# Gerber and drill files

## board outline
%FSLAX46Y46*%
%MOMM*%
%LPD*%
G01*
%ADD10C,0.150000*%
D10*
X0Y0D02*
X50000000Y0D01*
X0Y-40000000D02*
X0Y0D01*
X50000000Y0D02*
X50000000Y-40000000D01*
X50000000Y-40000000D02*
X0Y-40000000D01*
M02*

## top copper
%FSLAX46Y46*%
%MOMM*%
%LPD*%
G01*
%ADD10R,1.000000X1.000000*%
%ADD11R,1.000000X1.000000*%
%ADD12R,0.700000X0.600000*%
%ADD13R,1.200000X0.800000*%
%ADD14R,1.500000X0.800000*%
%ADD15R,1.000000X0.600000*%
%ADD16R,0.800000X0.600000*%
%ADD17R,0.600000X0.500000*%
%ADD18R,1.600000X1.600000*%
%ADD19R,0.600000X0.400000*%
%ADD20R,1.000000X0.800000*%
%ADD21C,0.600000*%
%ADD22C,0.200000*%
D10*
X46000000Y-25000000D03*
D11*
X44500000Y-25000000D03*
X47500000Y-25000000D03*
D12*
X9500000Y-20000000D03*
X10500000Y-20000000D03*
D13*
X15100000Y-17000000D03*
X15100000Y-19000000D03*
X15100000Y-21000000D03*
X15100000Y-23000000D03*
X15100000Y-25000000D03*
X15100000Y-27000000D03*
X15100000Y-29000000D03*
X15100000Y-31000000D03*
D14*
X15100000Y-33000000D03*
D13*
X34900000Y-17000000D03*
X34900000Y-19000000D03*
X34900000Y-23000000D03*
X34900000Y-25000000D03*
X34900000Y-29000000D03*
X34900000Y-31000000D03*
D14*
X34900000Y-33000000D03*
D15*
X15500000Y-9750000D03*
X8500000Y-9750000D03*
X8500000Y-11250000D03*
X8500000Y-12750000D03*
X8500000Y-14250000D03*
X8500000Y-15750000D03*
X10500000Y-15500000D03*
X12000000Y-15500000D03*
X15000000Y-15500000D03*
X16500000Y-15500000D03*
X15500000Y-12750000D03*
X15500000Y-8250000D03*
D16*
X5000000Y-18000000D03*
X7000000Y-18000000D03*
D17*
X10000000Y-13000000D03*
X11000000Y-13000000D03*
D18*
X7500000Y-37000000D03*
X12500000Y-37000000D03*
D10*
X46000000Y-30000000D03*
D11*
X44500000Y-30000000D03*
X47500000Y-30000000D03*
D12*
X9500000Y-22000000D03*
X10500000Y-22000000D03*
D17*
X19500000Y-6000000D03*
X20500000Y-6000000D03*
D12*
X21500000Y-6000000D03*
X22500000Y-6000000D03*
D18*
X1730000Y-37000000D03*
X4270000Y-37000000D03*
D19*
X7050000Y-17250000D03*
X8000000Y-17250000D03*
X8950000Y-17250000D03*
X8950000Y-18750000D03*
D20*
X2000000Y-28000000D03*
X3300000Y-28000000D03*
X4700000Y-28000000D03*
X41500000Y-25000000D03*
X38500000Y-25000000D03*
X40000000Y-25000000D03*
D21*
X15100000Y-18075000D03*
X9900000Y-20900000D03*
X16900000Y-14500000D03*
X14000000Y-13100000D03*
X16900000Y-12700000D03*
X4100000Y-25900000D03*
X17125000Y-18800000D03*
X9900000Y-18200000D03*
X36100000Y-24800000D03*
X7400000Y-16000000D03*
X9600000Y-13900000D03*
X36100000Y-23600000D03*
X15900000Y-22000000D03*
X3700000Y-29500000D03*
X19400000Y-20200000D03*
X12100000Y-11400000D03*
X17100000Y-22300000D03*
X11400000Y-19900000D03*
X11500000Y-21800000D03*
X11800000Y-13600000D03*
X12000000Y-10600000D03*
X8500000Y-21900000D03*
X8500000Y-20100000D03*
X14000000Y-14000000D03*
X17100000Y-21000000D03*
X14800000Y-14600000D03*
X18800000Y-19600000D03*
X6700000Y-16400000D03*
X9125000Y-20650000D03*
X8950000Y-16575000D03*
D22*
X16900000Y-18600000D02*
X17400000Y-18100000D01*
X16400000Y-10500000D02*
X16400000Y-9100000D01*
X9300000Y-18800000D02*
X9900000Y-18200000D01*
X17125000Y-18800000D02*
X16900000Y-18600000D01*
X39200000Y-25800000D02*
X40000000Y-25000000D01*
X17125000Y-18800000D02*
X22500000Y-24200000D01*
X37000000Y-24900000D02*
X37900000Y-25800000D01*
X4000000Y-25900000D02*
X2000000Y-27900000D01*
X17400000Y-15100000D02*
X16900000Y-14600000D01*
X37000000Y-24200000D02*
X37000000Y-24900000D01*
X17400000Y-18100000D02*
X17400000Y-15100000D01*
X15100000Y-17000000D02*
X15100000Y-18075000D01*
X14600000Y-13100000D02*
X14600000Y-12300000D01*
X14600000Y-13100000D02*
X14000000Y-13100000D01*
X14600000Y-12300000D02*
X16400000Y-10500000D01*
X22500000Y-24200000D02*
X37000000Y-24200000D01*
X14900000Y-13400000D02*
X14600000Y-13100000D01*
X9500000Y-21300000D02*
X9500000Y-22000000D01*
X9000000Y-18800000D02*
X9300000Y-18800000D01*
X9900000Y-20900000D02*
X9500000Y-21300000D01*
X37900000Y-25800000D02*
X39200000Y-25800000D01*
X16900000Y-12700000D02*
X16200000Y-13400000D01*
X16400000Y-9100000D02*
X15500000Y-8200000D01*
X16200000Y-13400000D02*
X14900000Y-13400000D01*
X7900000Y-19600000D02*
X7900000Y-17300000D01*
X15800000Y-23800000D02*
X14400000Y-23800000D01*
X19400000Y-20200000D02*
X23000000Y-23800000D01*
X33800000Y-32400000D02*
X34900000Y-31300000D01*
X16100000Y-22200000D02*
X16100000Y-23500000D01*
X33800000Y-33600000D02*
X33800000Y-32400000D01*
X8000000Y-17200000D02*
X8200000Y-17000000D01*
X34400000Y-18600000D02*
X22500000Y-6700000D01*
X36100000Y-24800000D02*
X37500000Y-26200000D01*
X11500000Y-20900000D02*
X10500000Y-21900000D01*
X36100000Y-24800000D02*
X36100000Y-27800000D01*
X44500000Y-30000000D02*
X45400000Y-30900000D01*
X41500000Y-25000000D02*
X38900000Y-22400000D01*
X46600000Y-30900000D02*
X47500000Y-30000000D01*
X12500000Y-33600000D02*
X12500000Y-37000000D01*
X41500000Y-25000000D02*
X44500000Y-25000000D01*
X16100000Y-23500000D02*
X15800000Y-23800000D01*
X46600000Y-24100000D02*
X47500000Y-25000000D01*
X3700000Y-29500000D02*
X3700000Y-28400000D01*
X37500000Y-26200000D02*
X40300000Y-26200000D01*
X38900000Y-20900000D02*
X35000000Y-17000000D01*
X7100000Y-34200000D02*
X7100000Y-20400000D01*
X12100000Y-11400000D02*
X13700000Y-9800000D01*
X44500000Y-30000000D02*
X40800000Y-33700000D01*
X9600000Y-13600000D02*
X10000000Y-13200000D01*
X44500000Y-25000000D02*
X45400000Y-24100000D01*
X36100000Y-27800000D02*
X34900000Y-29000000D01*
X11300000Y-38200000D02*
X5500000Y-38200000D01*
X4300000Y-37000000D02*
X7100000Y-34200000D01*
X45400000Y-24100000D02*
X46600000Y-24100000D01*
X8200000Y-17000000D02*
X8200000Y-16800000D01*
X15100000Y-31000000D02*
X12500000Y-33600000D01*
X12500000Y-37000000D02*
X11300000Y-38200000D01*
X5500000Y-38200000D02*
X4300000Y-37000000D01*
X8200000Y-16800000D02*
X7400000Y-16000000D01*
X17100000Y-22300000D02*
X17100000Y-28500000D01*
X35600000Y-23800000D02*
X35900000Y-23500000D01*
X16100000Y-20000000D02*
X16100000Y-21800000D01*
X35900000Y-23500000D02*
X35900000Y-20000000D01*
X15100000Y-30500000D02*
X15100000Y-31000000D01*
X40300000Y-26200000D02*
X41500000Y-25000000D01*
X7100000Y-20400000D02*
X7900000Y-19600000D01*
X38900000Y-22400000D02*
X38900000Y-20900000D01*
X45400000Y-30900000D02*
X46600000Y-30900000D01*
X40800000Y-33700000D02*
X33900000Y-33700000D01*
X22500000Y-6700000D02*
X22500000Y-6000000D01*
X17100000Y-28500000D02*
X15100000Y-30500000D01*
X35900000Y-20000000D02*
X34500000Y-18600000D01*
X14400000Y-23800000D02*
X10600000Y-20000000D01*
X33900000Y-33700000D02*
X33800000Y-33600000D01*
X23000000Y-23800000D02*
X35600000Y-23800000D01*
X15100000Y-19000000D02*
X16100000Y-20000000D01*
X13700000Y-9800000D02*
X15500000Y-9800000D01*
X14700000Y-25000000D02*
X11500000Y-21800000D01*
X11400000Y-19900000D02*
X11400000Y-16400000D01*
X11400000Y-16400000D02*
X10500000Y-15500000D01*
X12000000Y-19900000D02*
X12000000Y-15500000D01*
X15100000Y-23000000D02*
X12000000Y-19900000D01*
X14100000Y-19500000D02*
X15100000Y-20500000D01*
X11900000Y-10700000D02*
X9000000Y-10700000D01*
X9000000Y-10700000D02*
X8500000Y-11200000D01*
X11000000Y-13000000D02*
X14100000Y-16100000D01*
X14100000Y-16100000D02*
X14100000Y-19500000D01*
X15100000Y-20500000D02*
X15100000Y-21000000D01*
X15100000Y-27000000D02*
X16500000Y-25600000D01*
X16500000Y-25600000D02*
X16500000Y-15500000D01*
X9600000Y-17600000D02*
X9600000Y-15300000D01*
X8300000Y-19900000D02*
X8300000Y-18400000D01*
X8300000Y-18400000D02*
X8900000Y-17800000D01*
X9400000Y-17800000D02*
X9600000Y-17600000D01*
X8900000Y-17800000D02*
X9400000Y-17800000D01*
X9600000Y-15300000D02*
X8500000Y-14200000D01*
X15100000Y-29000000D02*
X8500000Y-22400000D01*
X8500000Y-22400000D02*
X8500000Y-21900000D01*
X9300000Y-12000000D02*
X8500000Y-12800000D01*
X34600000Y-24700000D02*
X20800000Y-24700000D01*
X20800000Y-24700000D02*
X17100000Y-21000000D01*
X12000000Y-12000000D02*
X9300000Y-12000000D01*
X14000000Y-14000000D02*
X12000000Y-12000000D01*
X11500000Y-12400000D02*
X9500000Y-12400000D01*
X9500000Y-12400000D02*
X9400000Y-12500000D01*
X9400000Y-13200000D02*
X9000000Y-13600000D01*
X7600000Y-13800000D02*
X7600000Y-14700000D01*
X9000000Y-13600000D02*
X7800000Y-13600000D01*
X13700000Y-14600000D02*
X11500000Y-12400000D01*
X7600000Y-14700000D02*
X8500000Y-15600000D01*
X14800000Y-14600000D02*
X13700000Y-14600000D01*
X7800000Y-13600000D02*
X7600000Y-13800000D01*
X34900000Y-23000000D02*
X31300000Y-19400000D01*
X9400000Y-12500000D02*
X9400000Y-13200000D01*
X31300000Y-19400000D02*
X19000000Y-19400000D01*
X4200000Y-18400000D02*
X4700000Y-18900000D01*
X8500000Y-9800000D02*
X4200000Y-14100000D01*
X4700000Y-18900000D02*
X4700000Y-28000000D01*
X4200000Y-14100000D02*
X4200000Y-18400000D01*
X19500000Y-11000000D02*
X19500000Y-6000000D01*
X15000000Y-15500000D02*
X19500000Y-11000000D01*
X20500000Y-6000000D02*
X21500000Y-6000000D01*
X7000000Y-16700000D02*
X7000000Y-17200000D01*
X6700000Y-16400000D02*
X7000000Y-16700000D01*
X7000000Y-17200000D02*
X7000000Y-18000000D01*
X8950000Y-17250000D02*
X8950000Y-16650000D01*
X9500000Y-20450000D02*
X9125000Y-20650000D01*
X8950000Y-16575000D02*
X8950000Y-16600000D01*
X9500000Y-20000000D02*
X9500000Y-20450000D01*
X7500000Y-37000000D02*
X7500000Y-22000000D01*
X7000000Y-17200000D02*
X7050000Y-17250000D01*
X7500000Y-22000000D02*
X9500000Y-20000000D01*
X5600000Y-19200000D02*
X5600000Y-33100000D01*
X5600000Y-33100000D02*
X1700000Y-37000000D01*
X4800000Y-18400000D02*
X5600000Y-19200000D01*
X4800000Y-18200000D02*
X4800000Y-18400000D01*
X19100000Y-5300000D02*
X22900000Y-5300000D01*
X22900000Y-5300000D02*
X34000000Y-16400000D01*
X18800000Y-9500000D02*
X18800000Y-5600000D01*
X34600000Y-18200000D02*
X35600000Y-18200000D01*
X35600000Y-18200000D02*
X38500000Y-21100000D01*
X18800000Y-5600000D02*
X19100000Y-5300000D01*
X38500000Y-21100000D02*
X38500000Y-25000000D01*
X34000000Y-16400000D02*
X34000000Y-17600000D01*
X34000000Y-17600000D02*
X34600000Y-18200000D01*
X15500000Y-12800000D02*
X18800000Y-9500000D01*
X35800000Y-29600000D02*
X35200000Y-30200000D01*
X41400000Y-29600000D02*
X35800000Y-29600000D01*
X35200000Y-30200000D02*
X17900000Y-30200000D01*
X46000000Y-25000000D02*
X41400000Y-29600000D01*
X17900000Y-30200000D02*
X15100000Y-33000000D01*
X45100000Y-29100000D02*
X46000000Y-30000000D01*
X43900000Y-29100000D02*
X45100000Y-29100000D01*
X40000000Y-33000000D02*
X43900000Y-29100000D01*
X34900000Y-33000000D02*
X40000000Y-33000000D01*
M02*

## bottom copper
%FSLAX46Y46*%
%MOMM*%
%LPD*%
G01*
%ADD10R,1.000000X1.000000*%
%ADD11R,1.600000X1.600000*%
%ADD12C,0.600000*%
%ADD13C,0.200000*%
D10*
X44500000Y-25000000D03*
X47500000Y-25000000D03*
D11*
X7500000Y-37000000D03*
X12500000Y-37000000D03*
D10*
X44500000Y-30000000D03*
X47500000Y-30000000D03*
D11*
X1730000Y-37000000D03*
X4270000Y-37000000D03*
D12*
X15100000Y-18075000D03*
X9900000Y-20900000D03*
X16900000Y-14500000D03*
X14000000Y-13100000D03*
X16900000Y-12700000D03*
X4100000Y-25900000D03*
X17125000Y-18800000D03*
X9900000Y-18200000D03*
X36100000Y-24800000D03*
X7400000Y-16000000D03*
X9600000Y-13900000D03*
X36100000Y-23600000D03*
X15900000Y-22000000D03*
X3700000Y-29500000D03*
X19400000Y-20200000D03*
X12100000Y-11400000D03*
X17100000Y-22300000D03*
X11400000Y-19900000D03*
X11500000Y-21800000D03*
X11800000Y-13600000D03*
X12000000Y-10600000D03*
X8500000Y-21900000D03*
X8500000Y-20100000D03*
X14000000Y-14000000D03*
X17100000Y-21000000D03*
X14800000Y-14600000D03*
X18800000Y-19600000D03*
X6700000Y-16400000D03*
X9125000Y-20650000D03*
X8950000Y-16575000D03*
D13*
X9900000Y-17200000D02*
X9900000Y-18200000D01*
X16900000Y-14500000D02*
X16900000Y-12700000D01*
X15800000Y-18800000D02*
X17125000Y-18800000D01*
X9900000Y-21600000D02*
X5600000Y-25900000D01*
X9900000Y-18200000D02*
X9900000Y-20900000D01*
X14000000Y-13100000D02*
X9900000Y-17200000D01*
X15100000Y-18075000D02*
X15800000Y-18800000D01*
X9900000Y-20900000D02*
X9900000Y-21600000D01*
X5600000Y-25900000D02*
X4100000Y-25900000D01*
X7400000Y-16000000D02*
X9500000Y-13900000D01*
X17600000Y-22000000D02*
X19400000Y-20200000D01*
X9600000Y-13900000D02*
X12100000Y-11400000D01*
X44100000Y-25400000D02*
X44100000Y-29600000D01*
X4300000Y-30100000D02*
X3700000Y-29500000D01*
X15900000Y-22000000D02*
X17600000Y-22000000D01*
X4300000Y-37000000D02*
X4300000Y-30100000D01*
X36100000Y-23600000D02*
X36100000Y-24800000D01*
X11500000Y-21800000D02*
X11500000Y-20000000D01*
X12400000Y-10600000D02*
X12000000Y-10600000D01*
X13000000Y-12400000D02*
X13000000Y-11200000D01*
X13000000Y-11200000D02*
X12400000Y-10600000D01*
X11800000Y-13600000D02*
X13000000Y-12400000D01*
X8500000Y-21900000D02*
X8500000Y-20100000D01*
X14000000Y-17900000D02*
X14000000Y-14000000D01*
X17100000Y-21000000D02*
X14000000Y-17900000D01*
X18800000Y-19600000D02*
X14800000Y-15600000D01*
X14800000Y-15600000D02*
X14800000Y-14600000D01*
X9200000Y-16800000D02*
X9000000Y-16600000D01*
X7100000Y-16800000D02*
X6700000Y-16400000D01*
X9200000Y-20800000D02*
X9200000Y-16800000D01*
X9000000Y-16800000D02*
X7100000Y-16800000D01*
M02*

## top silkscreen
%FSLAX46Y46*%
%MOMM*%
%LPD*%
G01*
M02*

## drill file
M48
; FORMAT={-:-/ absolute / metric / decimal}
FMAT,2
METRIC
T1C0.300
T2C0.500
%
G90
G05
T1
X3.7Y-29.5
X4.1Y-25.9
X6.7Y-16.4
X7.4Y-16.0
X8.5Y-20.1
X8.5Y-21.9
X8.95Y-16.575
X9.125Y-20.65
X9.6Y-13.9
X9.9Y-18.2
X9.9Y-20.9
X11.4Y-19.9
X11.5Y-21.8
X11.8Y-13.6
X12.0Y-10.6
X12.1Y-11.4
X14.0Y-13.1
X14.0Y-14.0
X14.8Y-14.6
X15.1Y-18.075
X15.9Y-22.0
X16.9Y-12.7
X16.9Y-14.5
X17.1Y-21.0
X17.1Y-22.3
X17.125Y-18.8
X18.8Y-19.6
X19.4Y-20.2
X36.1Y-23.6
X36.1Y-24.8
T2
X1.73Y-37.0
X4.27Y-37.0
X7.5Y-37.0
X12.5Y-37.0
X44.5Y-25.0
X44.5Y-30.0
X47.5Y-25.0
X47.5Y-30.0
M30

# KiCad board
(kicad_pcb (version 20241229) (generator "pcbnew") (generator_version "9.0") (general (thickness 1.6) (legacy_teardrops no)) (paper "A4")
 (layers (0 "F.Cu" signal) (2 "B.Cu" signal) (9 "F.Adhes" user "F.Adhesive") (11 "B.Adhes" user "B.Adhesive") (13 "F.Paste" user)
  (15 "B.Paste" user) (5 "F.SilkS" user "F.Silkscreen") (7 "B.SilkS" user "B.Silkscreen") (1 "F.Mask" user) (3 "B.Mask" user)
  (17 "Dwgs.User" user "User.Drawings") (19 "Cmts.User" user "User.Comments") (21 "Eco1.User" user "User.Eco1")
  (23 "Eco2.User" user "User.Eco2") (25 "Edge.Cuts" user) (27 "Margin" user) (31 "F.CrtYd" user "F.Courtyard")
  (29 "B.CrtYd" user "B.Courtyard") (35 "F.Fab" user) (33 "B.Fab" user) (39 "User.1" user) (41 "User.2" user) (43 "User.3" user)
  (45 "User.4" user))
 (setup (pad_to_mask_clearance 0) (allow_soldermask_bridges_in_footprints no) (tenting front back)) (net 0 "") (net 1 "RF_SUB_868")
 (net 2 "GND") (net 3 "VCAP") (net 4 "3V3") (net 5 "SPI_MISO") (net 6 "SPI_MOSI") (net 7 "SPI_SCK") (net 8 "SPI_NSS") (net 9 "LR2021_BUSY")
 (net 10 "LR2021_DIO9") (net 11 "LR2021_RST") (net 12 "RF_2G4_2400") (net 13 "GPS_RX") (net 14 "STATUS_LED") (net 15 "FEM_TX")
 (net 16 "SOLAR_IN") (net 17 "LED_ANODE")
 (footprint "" (layer "F.Cu") (at 46 25)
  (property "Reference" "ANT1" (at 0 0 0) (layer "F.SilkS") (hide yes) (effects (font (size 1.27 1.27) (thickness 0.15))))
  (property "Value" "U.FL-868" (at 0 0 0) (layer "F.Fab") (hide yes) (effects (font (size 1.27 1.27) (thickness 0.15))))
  (pad "1" smd rect (at 0 0) (size 1 1) (layers "F.Cu" "F.Mask") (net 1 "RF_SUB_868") (thermal_bridge_angle 45))
  (pad "2" thru_hole rect (at -1.5 0) (size 1 1) (drill 0.5) (layers "*.Cu" "*.Mask") (remove_unused_layers no) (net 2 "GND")
   (thermal_bridge_angle 45))
  (pad "3" thru_hole rect (at 1.5 0) (size 1 1) (drill 0.5) (layers "*.Cu" "*.Mask") (remove_unused_layers no) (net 2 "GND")
   (thermal_bridge_angle 45)))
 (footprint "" (layer "F.Cu") (at 10 20)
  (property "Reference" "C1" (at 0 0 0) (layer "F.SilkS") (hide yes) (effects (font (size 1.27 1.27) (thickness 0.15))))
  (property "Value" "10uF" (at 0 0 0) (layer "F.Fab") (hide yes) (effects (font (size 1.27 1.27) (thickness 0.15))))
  (pad "1" smd rect (at -0.5 0) (size 0.7 0.6) (layers "F.Cu" "F.Mask") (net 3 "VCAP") (thermal_bridge_angle 45))
  (pad "2" smd rect (at 0.5 0) (size 0.7 0.6) (layers "F.Cu" "F.Mask") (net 2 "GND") (thermal_bridge_angle 45)))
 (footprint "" (layer "F.Cu") (at 25 25)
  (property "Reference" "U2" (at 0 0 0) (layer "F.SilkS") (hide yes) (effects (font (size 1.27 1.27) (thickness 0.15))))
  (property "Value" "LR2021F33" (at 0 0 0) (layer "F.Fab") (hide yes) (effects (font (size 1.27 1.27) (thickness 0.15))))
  (pad "1" smd rect (at -9.9 -8) (size 1.2 0.8) (layers "F.Cu" "F.Mask") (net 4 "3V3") (thermal_bridge_angle 45))
  (pad "2" smd rect (at -9.9 -6) (size 1.2 0.8) (layers "F.Cu" "F.Mask") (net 2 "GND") (thermal_bridge_angle 45))
  (pad "3" smd rect (at -9.9 -4) (size 1.2 0.8) (layers "F.Cu" "F.Mask") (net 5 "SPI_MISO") (thermal_bridge_angle 45))
  (pad "4" smd rect (at -9.9 -2) (size 1.2 0.8) (layers "F.Cu" "F.Mask") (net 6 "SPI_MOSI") (thermal_bridge_angle 45))
  (pad "5" smd rect (at -9.9 0) (size 1.2 0.8) (layers "F.Cu" "F.Mask") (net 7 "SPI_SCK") (thermal_bridge_angle 45))
  (pad "6" smd rect (at -9.9 2) (size 1.2 0.8) (layers "F.Cu" "F.Mask") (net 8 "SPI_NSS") (thermal_bridge_angle 45))
  (pad "7" smd rect (at -9.9 4) (size 1.2 0.8) (layers "F.Cu" "F.Mask") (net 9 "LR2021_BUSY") (thermal_bridge_angle 45))
  (pad "8" smd rect (at -9.9 6) (size 1.2 0.8) (layers "F.Cu" "F.Mask") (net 2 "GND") (thermal_bridge_angle 45))
  (pad "9" smd rect (at -9.9 8) (size 1.5 0.8) (layers "F.Cu" "F.Mask") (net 1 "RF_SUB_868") (thermal_bridge_angle 45))
  (pad "10" smd rect (at 9.9 -8) (size 1.2 0.8) (layers "F.Cu" "F.Mask") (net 2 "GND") (thermal_bridge_angle 45))
  (pad "11" smd rect (at 9.9 -6) (size 1.2 0.8) (layers "F.Cu" "F.Mask") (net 2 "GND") (thermal_bridge_angle 45))
  (pad "13" smd rect (at 9.9 -2) (size 1.2 0.8) (layers "F.Cu" "F.Mask") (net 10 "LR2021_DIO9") (thermal_bridge_angle 45))
  (pad "14" smd rect (at 9.9 0) (size 1.2 0.8) (layers "F.Cu" "F.Mask") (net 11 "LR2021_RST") (thermal_bridge_angle 45))
  (pad "16" smd rect (at 9.9 4) (size 1.2 0.8) (layers "F.Cu" "F.Mask") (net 2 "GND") (thermal_bridge_angle 45))
  (pad "17" smd rect (at 9.9 6) (size 1.2 0.8) (layers "F.Cu" "F.Mask") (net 2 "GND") (thermal_bridge_angle 45))
  (pad "18" smd rect (at 9.9 8) (size 1.5 0.8) (layers "F.Cu" "F.Mask") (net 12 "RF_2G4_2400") (thermal_bridge_angle 45)))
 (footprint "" (layer "F.Cu") (at 12 12)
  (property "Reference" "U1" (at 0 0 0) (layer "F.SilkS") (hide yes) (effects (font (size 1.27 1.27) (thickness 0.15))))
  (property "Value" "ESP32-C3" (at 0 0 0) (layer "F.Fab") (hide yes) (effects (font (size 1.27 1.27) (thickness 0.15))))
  (pad "GND" smd rect (at 3.5 -2.25) (size 1 0.6) (layers "F.Cu" "F.Mask") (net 2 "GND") (thermal_bridge_angle 45))
  (pad "GPIO1" smd rect (at -3.5 -2.25) (size 1 0.6) (layers "F.Cu" "F.Mask") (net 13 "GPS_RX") (thermal_bridge_angle 45))
  (pad "GPIO2" smd rect (at -3.5 -0.75) (size 1 0.6) (layers "F.Cu" "F.Mask") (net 5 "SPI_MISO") (thermal_bridge_angle 45))
  (pad "GPIO3" smd rect (at -3.5 0.75) (size 1 0.6) (layers "F.Cu" "F.Mask") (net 11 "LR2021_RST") (thermal_bridge_angle 45))
  (pad "GPIO4" smd rect (at -3.5 2.25) (size 1 0.6) (layers "F.Cu" "F.Mask") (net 9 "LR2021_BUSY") (thermal_bridge_angle 45))
  (pad "GPIO5" smd rect (at -3.5 3.75) (size 1 0.6) (layers "F.Cu" "F.Mask") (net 10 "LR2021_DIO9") (thermal_bridge_angle 45))
  (pad "GPIO6" smd rect (at -1.5 3.5) (size 1 0.6) (layers "F.Cu" "F.Mask") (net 7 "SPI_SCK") (thermal_bridge_angle 45))
  (pad "GPIO7" smd rect (at 0 3.5) (size 1 0.6) (layers "F.Cu" "F.Mask") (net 6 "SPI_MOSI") (thermal_bridge_angle 45))
  (pad "GPIO9" smd rect (at 3 3.5) (size 1 0.6) (layers "F.Cu" "F.Mask") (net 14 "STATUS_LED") (thermal_bridge_angle 45))
  (pad "GPIO10" smd rect (at 4.5 3.5) (size 1 0.6) (layers "F.Cu" "F.Mask") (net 8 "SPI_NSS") (thermal_bridge_angle 45))
  (pad "GPIO19" smd rect (at 3.5 0.75) (size 1 0.6) (layers "F.Cu" "F.Mask") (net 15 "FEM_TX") (thermal_bridge_angle 45))
  (pad "VCC" smd rect (at 3.5 -3.75) (size 1 0.6) (layers "F.Cu" "F.Mask") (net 4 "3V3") (thermal_bridge_angle 45)))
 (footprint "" (layer "F.Cu") (at 6 18)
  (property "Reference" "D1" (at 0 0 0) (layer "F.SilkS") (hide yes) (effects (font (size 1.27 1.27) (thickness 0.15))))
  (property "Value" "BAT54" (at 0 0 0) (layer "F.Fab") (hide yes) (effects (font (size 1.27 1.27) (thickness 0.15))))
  (pad "A" smd rect (at -1 0) (size 0.8 0.6) (layers "F.Cu" "F.Mask") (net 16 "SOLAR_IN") (thermal_bridge_angle 45))
  (pad "K" smd rect (at 1 0) (size 0.8 0.6) (layers "F.Cu" "F.Mask") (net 3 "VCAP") (thermal_bridge_angle 45)))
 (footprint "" (layer "F.Cu") (at 10.5 13)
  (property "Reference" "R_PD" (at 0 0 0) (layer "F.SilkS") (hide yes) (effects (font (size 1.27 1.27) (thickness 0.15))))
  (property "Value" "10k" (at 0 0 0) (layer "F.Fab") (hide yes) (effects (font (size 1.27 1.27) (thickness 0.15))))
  (pad "1" smd rect (at -0.5 0) (size 0.6 0.5) (layers "F.Cu" "F.Mask") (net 2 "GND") (thermal_bridge_angle 45))
  (pad "2" smd rect (at 0.5 0) (size 0.6 0.5) (layers "F.Cu" "F.Mask") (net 5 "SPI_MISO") (thermal_bridge_angle 45)))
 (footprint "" (layer "F.Cu") (at 10 37)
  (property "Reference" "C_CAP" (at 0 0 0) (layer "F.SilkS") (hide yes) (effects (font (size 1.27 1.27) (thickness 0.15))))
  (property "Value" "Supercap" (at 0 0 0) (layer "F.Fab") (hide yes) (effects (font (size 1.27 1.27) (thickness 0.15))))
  (pad "1" thru_hole rect (at -2.5 0) (size 1.6 1.6) (drill 0.5) (layers "*.Cu" "*.Mask") (remove_unused_layers no) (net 3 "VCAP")
   (thermal_bridge_angle 45))
  (pad "2" thru_hole rect (at 2.5 0) (size 1.6 1.6) (drill 0.5) (layers "*.Cu" "*.Mask") (remove_unused_layers no) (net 2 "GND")
   (thermal_bridge_angle 45)))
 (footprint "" (layer "F.Cu") (at 46 30)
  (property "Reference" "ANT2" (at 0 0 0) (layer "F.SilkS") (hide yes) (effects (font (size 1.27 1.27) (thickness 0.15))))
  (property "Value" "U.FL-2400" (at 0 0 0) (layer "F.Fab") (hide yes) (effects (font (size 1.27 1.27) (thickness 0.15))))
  (pad "1" smd rect (at 0 0) (size 1 1) (layers "F.Cu" "F.Mask") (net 12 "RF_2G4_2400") (thermal_bridge_angle 45))
  (pad "2" thru_hole rect (at -1.5 0) (size 1 1) (drill 0.5) (layers "*.Cu" "*.Mask") (remove_unused_layers no) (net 2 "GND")
   (thermal_bridge_angle 45))
  (pad "3" thru_hole rect (at 1.5 0) (size 1 1) (drill 0.5) (layers "*.Cu" "*.Mask") (remove_unused_layers no) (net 2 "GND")
   (thermal_bridge_angle 45)))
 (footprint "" (layer "F.Cu") (at 10 22)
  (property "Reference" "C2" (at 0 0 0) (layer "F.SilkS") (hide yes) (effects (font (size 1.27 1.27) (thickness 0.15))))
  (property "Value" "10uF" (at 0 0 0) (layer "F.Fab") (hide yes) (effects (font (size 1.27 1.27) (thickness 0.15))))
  (pad "1" smd rect (at -0.5 0) (size 0.7 0.6) (layers "F.Cu" "F.Mask") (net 4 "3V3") (thermal_bridge_angle 45))
  (pad "2" smd rect (at 0.5 0) (size 0.7 0.6) (layers "F.Cu" "F.Mask") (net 2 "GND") (thermal_bridge_angle 45)))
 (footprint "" (layer "F.Cu") (at 20 6)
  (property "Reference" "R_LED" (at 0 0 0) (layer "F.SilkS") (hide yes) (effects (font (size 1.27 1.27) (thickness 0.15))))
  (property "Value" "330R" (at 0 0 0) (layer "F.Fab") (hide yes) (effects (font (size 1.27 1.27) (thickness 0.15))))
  (pad "1" smd rect (at -0.5 0) (size 0.6 0.5) (layers "F.Cu" "F.Mask") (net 14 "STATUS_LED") (thermal_bridge_angle 45))
  (pad "2" smd rect (at 0.5 0) (size 0.6 0.5) (layers "F.Cu" "F.Mask") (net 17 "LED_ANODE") (thermal_bridge_angle 45)))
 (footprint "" (layer "F.Cu") (at 22 6)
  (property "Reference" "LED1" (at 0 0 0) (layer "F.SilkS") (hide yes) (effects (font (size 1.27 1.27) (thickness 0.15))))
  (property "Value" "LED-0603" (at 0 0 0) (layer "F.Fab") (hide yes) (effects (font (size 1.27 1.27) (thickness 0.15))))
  (pad "A" smd rect (at -0.5 0) (size 0.7 0.6) (layers "F.Cu" "F.Mask") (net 17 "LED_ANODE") (thermal_bridge_angle 45))
  (pad "K" smd rect (at 0.5 0) (size 0.7 0.6) (layers "F.Cu" "F.Mask") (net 2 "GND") (thermal_bridge_angle 45)))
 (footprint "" (layer "F.Cu") (at 3 37)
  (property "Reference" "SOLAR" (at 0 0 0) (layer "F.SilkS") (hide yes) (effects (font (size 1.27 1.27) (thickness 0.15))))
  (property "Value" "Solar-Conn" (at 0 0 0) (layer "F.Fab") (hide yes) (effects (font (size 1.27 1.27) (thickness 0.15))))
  (pad "1" thru_hole rect (at -1.27 0) (size 1.6 1.6) (drill 0.5) (layers "*.Cu" "*.Mask") (remove_unused_layers no) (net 16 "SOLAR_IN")
   (thermal_bridge_angle 45))
  (pad "2" thru_hole rect (at 1.27 0) (size 1.6 1.6) (drill 0.5) (layers "*.Cu" "*.Mask") (remove_unused_layers no) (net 2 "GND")
   (thermal_bridge_angle 45)))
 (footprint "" (layer "F.Cu") (at 8 18)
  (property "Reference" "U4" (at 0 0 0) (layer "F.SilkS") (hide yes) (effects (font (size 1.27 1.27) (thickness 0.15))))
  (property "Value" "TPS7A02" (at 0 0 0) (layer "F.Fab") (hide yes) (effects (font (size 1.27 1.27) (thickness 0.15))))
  (pad "1" smd rect (at -0.95 -0.75) (size 0.6 0.4) (layers "F.Cu" "F.Mask") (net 3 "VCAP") (thermal_bridge_angle 45))
  (pad "2" smd rect (at 0 -0.75) (size 0.6 0.4) (layers "F.Cu" "F.Mask") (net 2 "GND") (thermal_bridge_angle 45))
  (pad "3" smd rect (at 0.95 -0.75) (size 0.6 0.4) (layers "F.Cu" "F.Mask") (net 3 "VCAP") (thermal_bridge_angle 45))
  (pad "4" smd rect (at 0.95 0.75) (size 0.6 0.4) (layers "F.Cu" "F.Mask") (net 4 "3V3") (thermal_bridge_angle 45)))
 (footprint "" (layer "F.Cu") (at 4 28)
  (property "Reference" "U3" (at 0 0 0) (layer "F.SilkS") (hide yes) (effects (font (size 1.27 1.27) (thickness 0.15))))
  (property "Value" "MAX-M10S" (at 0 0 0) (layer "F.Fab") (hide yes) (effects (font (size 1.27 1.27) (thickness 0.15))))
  (pad "1" smd rect (at -2 0) (size 1 0.8) (layers "F.Cu" "F.Mask") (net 4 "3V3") (thermal_bridge_angle 45))
  (pad "2" smd rect (at -0.7 0) (size 1 0.8) (layers "F.Cu" "F.Mask") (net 2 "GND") (thermal_bridge_angle 45))
  (pad "3" smd rect (at 0.7 0) (size 1 0.8) (layers "F.Cu" "F.Mask") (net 13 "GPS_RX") (thermal_bridge_angle 45)))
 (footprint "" (layer "F.Cu") (at 40 25)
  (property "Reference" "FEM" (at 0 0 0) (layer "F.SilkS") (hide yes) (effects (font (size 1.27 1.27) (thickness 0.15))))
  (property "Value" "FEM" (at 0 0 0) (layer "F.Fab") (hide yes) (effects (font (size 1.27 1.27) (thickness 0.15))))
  (pad "GND" smd rect (at 1.5 0) (size 1 0.8) (layers "F.Cu" "F.Mask") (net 2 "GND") (thermal_bridge_angle 45))
  (pad "TX" smd rect (at -1.5 0) (size 1 0.8) (layers "F.Cu" "F.Mask") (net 15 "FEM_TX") (thermal_bridge_angle 45))
  (pad "VCC" smd rect (at 0 0) (size 1 0.8) (layers "F.Cu" "F.Mask") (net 4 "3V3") (thermal_bridge_angle 45)))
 (gr_line (start 0 0) (end 50 0) (stroke (width 0.15) (type default)) (layer "Edge.Cuts"))
 (gr_line (start 0 40) (end 0 0) (stroke (width 0.15) (type default)) (layer "Edge.Cuts"))
 (gr_line (start 50 0) (end 50 40) (stroke (width 0.15) (type default)) (layer "Edge.Cuts"))
 (gr_line (start 50 40) (end 0 40) (stroke (width 0.15) (type default)) (layer "Edge.Cuts"))
 (segment (start 16.9 18.6) (end 17.4 18.1) (width 0.2) (layer "F.Cu") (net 4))
 (segment (start 16.4 10.5) (end 16.4 9.1) (width 0.2) (layer "F.Cu") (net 4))
 (segment (start 9.3 18.8) (end 9.9 18.2) (width 0.2) (layer "F.Cu") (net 4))
 (segment (start 17.125 18.8) (end 16.9 18.6) (width 0.2) (layer "F.Cu") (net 4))
 (segment (start 39.2 25.8) (end 40 25) (width 0.2) (layer "F.Cu") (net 4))
 (segment (start 17.125 18.8) (end 22.5 24.2) (width 0.2) (layer "F.Cu") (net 4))
 (segment (start 37 24.9) (end 37.9 25.8) (width 0.2) (layer "F.Cu") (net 4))
 (segment (start 4 25.9) (end 2 27.9) (width 0.2) (layer "F.Cu") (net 4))
 (segment (start 17.4 15.1) (end 16.9 14.6) (width 0.2) (layer "F.Cu") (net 4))
 (segment (start 37 24.2) (end 37 24.9) (width 0.2) (layer "F.Cu") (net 4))
 (segment (start 17.4 18.1) (end 17.4 15.1) (width 0.2) (layer "F.Cu") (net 4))
 (segment (start 15.1 17) (end 15.1 18.075) (width 0.2) (layer "F.Cu") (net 4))
 (segment (start 14.6 13.1) (end 14.6 12.3) (width 0.2) (layer "F.Cu") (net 4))
 (segment (start 14.6 13.1) (end 14 13.1) (width 0.2) (layer "F.Cu") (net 4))
 (segment (start 14.6 12.3) (end 16.4 10.5) (width 0.2) (layer "F.Cu") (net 4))
 (segment (start 22.5 24.2) (end 37 24.2) (width 0.2) (layer "F.Cu") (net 4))
 (segment (start 14.9 13.4) (end 14.6 13.1) (width 0.2) (layer "F.Cu") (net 4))
 (segment (start 9.5 21.3) (end 9.5 22) (width 0.2) (layer "F.Cu") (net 4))
 (segment (start 9 18.8) (end 9.3 18.8) (width 0.2) (layer "F.Cu") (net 4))
 (segment (start 9.9 20.9) (end 9.5 21.3) (width 0.2) (layer "F.Cu") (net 4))
 (segment (start 37.9 25.8) (end 39.2 25.8) (width 0.2) (layer "F.Cu") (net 4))
 (segment (start 16.9 12.7) (end 16.2 13.4) (width 0.2) (layer "F.Cu") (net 4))
 (segment (start 16.4 9.1) (end 15.5 8.2) (width 0.2) (layer "F.Cu") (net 4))
 (segment (start 16.2 13.4) (end 14.9 13.4) (width 0.2) (layer "F.Cu") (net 4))
 (via (at 15.1 18.075) (size 0.6) (drill 0.3) (layers "F.Cu" "B.Cu") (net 4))
 (via (at 9.9 20.9) (size 0.6) (drill 0.3) (layers "F.Cu" "B.Cu") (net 4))
 (via (at 16.9 14.5) (size 0.6) (drill 0.3) (layers "F.Cu" "B.Cu") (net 4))
 (via (at 14 13.1) (size 0.6) (drill 0.3) (layers "F.Cu" "B.Cu") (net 4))
 (via (at 16.9 12.7) (size 0.6) (drill 0.3) (layers "F.Cu" "B.Cu") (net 4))
 (via (at 4.1 25.9) (size 0.6) (drill 0.3) (layers "F.Cu" "B.Cu") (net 4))
 (via (at 17.125 18.8) (size 0.6) (drill 0.3) (layers "F.Cu" "B.Cu") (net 4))
 (via (at 9.9 18.2) (size 0.6) (drill 0.3) (layers "F.Cu" "B.Cu") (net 4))
 (segment (start 9.9 17.2) (end 9.9 18.2) (width 0.2) (layer "B.Cu") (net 4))
 (segment (start 16.9 14.5) (end 16.9 12.7) (width 0.2) (layer "B.Cu") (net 4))
 (segment (start 15.8 18.8) (end 17.125 18.8) (width 0.2) (layer "B.Cu") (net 4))
 (segment (start 9.9 21.6) (end 5.6 25.9) (width 0.2) (layer "B.Cu") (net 4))
 (segment (start 9.9 18.2) (end 9.9 20.9) (width 0.2) (layer "B.Cu") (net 4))
 (segment (start 14 13.1) (end 9.9 17.2) (width 0.2) (layer "B.Cu") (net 4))
 (segment (start 15.1 18.075) (end 15.8 18.8) (width 0.2) (layer "B.Cu") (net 4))
 (segment (start 9.9 20.9) (end 9.9 21.6) (width 0.2) (layer "B.Cu") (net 4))
 (segment (start 5.6 25.9) (end 4.1 25.9) (width 0.2) (layer "B.Cu") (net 4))
 (segment (start 7.9 19.6) (end 7.9 17.3) (width 0.2) (layer "F.Cu") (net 2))
 (segment (start 15.8 23.8) (end 14.4 23.8) (width 0.2) (layer "F.Cu") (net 2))
 (segment (start 19.4 20.2) (end 23 23.8) (width 0.2) (layer "F.Cu") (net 2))
 (segment (start 33.8 32.4) (end 34.9 31.3) (width 0.2) (layer "F.Cu") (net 2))
 (segment (start 16.1 22.2) (end 16.1 23.5) (width 0.2) (layer "F.Cu") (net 2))
 (segment (start 33.8 33.6) (end 33.8 32.4) (width 0.2) (layer "F.Cu") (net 2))
 (segment (start 8 17.2) (end 8.2 17) (width 0.2) (layer "F.Cu") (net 2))
 (segment (start 34.4 18.6) (end 22.5 6.7) (width 0.2) (layer "F.Cu") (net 2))
 (segment (start 36.1 24.8) (end 37.5 26.2) (width 0.2) (layer "F.Cu") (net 2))
 (segment (start 11.5 20.9) (end 10.5 21.9) (width 0.2) (layer "F.Cu") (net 2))
 (segment (start 36.1 24.8) (end 36.1 27.8) (width 0.2) (layer "F.Cu") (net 2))
 (segment (start 44.5 30) (end 45.4 30.9) (width 0.2) (layer "F.Cu") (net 2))
 (segment (start 41.5 25) (end 38.9 22.4) (width 0.2) (layer "F.Cu") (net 2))
 (segment (start 46.6 30.9) (end 47.5 30) (width 0.2) (layer "F.Cu") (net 2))
 (segment (start 12.5 33.6) (end 12.5 37) (width 0.2) (layer "F.Cu") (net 2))
 (segment (start 41.5 25) (end 44.5 25) (width 0.2) (layer "F.Cu") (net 2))
 (segment (start 16.1 23.5) (end 15.8 23.8) (width 0.2) (layer "F.Cu") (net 2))
 (segment (start 46.6 24.1) (end 47.5 25) (width 0.2) (layer "F.Cu") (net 2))
 (segment (start 3.7 29.5) (end 3.7 28.4) (width 0.2) (layer "F.Cu") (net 2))
 (segment (start 37.5 26.2) (end 40.3 26.2) (width 0.2) (layer "F.Cu") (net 2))
 (segment (start 38.9 20.9) (end 35 17) (width 0.2) (layer "F.Cu") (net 2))
 (segment (start 7.1 34.2) (end 7.1 20.4) (width 0.2) (layer "F.Cu") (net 2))
 (segment (start 12.1 11.4) (end 13.7 9.8) (width 0.2) (layer "F.Cu") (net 2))
 (segment (start 44.5 30) (end 40.8 33.7) (width 0.2) (layer "F.Cu") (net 2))
 (segment (start 9.6 13.6) (end 10 13.2) (width 0.2) (layer "F.Cu") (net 2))
 (segment (start 44.5 25) (end 45.4 24.1) (width 0.2) (layer "F.Cu") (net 2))
 (segment (start 36.1 27.8) (end 34.9 29) (width 0.2) (layer "F.Cu") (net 2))
 (segment (start 11.3 38.2) (end 5.5 38.2) (width 0.2) (layer "F.Cu") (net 2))
 (segment (start 4.3 37) (end 7.1 34.2) (width 0.2) (layer "F.Cu") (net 2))
 (segment (start 45.4 24.1) (end 46.6 24.1) (width 0.2) (layer "F.Cu") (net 2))
 (segment (start 8.2 17) (end 8.2 16.8) (width 0.2) (layer "F.Cu") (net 2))
 (segment (start 15.1 31) (end 12.5 33.6) (width 0.2) (layer "F.Cu") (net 2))
 (segment (start 12.5 37) (end 11.3 38.2) (width 0.2) (layer "F.Cu") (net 2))
 (segment (start 5.5 38.2) (end 4.3 37) (width 0.2) (layer "F.Cu") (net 2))
 (segment (start 8.2 16.8) (end 7.4 16) (width 0.2) (layer "F.Cu") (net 2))
 (segment (start 17.1 22.3) (end 17.1 28.5) (width 0.2) (layer "F.Cu") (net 2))
 (segment (start 35.6 23.8) (end 35.9 23.5) (width 0.2) (layer "F.Cu") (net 2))
 (segment (start 16.1 20) (end 16.1 21.8) (width 0.2) (layer "F.Cu") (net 2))
 (segment (start 35.9 23.5) (end 35.9 20) (width 0.2) (layer "F.Cu") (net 2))
 (segment (start 15.1 30.5) (end 15.1 31) (width 0.2) (layer "F.Cu") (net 2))
 (segment (start 40.3 26.2) (end 41.5 25) (width 0.2) (layer "F.Cu") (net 2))
 (segment (start 7.1 20.4) (end 7.9 19.6) (width 0.2) (layer "F.Cu") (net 2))
 (segment (start 38.9 22.4) (end 38.9 20.9) (width 0.2) (layer "F.Cu") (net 2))
 (segment (start 45.4 30.9) (end 46.6 30.9) (width 0.2) (layer "F.Cu") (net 2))
 (segment (start 40.8 33.7) (end 33.9 33.7) (width 0.2) (layer "F.Cu") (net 2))
 (segment (start 22.5 6.7) (end 22.5 6) (width 0.2) (layer "F.Cu") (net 2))
 (segment (start 17.1 28.5) (end 15.1 30.5) (width 0.2) (layer "F.Cu") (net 2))
 (segment (start 35.9 20) (end 34.5 18.6) (width 0.2) (layer "F.Cu") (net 2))
 (segment (start 14.4 23.8) (end 10.6 20) (width 0.2) (layer "F.Cu") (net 2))
 (segment (start 33.9 33.7) (end 33.8 33.6) (width 0.2) (layer "F.Cu") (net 2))
 (segment (start 23 23.8) (end 35.6 23.8) (width 0.2) (layer "F.Cu") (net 2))
 (segment (start 15.1 19) (end 16.1 20) (width 0.2) (layer "F.Cu") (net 2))
 (segment (start 13.7 9.8) (end 15.5 9.8) (width 0.2) (layer "F.Cu") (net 2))
 (via (at 36.1 24.8) (size 0.6) (drill 0.3) (layers "F.Cu" "B.Cu") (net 2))
 (via (at 7.4 16) (size 0.6) (drill 0.3) (layers "F.Cu" "B.Cu") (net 2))
 (via (at 9.6 13.9) (size 0.6) (drill 0.3) (layers "F.Cu" "B.Cu") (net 2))
 (via (at 36.1 23.6) (size 0.6) (drill 0.3) (layers "F.Cu" "B.Cu") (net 2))
 (via (at 15.9 22) (size 0.6) (drill 0.3) (layers "F.Cu" "B.Cu") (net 2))
 (via (at 3.7 29.5) (size 0.6) (drill 0.3) (layers "F.Cu" "B.Cu") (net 2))
 (via (at 19.4 20.2) (size 0.6) (drill 0.3) (layers "F.Cu" "B.Cu") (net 2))
 (via (at 12.1 11.4) (size 0.6) (drill 0.3) (layers "F.Cu" "B.Cu") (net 2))
 (via (at 17.1 22.3) (size 0.6) (drill 0.3) (layers "F.Cu" "B.Cu") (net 2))
 (segment (start 7.4 16) (end 9.5 13.9) (width 0.2) (layer "B.Cu") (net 2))
 (segment (start 17.6 22) (end 19.4 20.2) (width 0.2) (layer "B.Cu") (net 2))
 (segment (start 9.6 13.9) (end 12.1 11.4) (width 0.2) (layer "B.Cu") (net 2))
 (segment (start 44.1 25.4) (end 44.1 29.6) (width 0.2) (layer "B.Cu") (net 2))
 (segment (start 4.3 30.1) (end 3.7 29.5) (width 0.2) (layer "B.Cu") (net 2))
 (segment (start 15.9 22) (end 17.6 22) (width 0.2) (layer "B.Cu") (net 2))
 (segment (start 4.3 37) (end 4.3 30.1) (width 0.2) (layer "B.Cu") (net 2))
 (segment (start 36.1 23.6) (end 36.1 24.8) (width 0.2) (layer "B.Cu") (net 2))
 (segment (start 14.7 25) (end 11.5 21.8) (width 0.2) (layer "F.Cu") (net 7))
 (segment (start 11.4 19.9) (end 11.4 16.4) (width 0.2) (layer "F.Cu") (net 7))
 (segment (start 11.4 16.4) (end 10.5 15.5) (width 0.2) (layer "F.Cu") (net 7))
 (via (at 11.4 19.9) (size 0.6) (drill 0.3) (layers "F.Cu" "B.Cu") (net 7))
 (via (at 11.5 21.8) (size 0.6) (drill 0.3) (layers "F.Cu" "B.Cu") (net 7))
 (segment (start 11.5 21.8) (end 11.5 20) (width 0.2) (layer "B.Cu") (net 7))
 (segment (start 12 19.9) (end 12 15.5) (width 0.2) (layer "F.Cu") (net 6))
 (segment (start 15.1 23) (end 12 19.9) (width 0.2) (layer "F.Cu") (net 6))
 (segment (start 14.1 19.5) (end 15.1 20.5) (width 0.2) (layer "F.Cu") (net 5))
 (segment (start 11.9 10.7) (end 9 10.7) (width 0.2) (layer "F.Cu") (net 5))
 (segment (start 9 10.7) (end 8.5 11.2) (width 0.2) (layer "F.Cu") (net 5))
 (segment (start 11 13) (end 14.1 16.1) (width 0.2) (layer "F.Cu") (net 5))
 (segment (start 14.1 16.1) (end 14.1 19.5) (width 0.2) (layer "F.Cu") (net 5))
 (segment (start 15.1 20.5) (end 15.1 21) (width 0.2) (layer "F.Cu") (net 5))
 (via (at 11.8 13.6) (size 0.6) (drill 0.3) (layers "F.Cu" "B.Cu") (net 5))
 (via (at 12 10.6) (size 0.6) (drill 0.3) (layers "F.Cu" "B.Cu") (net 5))
 (segment (start 12.4 10.6) (end 12 10.6) (width 0.2) (layer "B.Cu") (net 5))
 (segment (start 13 12.4) (end 13 11.2) (width 0.2) (layer "B.Cu") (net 5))
 (segment (start 13 11.2) (end 12.4 10.6) (width 0.2) (layer "B.Cu") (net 5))
 (segment (start 11.8 13.6) (end 13 12.4) (width 0.2) (layer "B.Cu") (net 5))
 (segment (start 15.1 27) (end 16.5 25.6) (width 0.2) (layer "F.Cu") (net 8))
 (segment (start 16.5 25.6) (end 16.5 15.5) (width 0.2) (layer "F.Cu") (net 8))
 (segment (start 9.6 17.6) (end 9.6 15.3) (width 0.2) (layer "F.Cu") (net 9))
 (segment (start 8.3 19.9) (end 8.3 18.4) (width 0.2) (layer "F.Cu") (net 9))
 (segment (start 8.3 18.4) (end 8.9 17.8) (width 0.2) (layer "F.Cu") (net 9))
 (segment (start 9.4 17.8) (end 9.6 17.6) (width 0.2) (layer "F.Cu") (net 9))
 (segment (start 8.9 17.8) (end 9.4 17.8) (width 0.2) (layer "F.Cu") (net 9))
 (segment (start 9.6 15.3) (end 8.5 14.2) (width 0.2) (layer "F.Cu") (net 9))
 (segment (start 15.1 29) (end 8.5 22.4) (width 0.2) (layer "F.Cu") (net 9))
 (segment (start 8.5 22.4) (end 8.5 21.9) (width 0.2) (layer "F.Cu") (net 9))
 (via (at 8.5 21.9) (size 0.6) (drill 0.3) (layers "F.Cu" "B.Cu") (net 9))
 (via (at 8.5 20.1) (size 0.6) (drill 0.3) (layers "F.Cu" "B.Cu") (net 9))
 (segment (start 8.5 21.9) (end 8.5 20.1) (width 0.2) (layer "B.Cu") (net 9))
 (segment (start 9.3 12) (end 8.5 12.8) (width 0.2) (layer "F.Cu") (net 11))
 (segment (start 34.6 24.7) (end 20.8 24.7) (width 0.2) (layer "F.Cu") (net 11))
 (segment (start 20.8 24.7) (end 17.1 21) (width 0.2) (layer "F.Cu") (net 11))
 (segment (start 12 12) (end 9.3 12) (width 0.2) (layer "F.Cu") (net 11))
 (segment (start 14 14) (end 12 12) (width 0.2) (layer "F.Cu") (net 11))
 (via (at 14 14) (size 0.6) (drill 0.3) (layers "F.Cu" "B.Cu") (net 11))
 (via (at 17.1 21) (size 0.6) (drill 0.3) (layers "F.Cu" "B.Cu") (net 11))
 (segment (start 14 17.9) (end 14 14) (width 0.2) (layer "B.Cu") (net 11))
 (segment (start 17.1 21) (end 14 17.9) (width 0.2) (layer "B.Cu") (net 11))
 (segment (start 11.5 12.4) (end 9.5 12.4) (width 0.2) (layer "F.Cu") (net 10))
 (segment (start 9.5 12.4) (end 9.4 12.5) (width 0.2) (layer "F.Cu") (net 10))
 (segment (start 9.4 13.2) (end 9 13.6) (width 0.2) (layer "F.Cu") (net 10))
 (segment (start 7.6 13.8) (end 7.6 14.7) (width 0.2) (layer "F.Cu") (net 10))
 (segment (start 9 13.6) (end 7.8 13.6) (width 0.2) (layer "F.Cu") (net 10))
 (segment (start 13.7 14.6) (end 11.5 12.4) (width 0.2) (layer "F.Cu") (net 10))
 (segment (start 7.6 14.7) (end 8.5 15.6) (width 0.2) (layer "F.Cu") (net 10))
 (segment (start 14.8 14.6) (end 13.7 14.6) (width 0.2) (layer "F.Cu") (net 10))
 (segment (start 7.8 13.6) (end 7.6 13.8) (width 0.2) (layer "F.Cu") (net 10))
 (segment (start 34.9 23) (end 31.3 19.4) (width 0.2) (layer "F.Cu") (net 10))
 (segment (start 9.4 12.5) (end 9.4 13.2) (width 0.2) (layer "F.Cu") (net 10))
 (segment (start 31.3 19.4) (end 19 19.4) (width 0.2) (layer "F.Cu") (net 10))
 (via (at 14.8 14.6) (size 0.6) (drill 0.3) (layers "F.Cu" "B.Cu") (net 10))
 (via (at 18.8 19.6) (size 0.6) (drill 0.3) (layers "F.Cu" "B.Cu") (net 10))
 (segment (start 18.8 19.6) (end 14.8 15.6) (width 0.2) (layer "B.Cu") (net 10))
 (segment (start 14.8 15.6) (end 14.8 14.6) (width 0.2) (layer "B.Cu") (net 10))
 (segment (start 4.2 18.4) (end 4.7 18.9) (width 0.2) (layer "F.Cu") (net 13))
 (segment (start 8.5 9.8) (end 4.2 14.1) (width 0.2) (layer "F.Cu") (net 13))
 (segment (start 4.7 18.9) (end 4.7 28) (width 0.2) (layer "F.Cu") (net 13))
 (segment (start 4.2 14.1) (end 4.2 18.4) (width 0.2) (layer "F.Cu") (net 13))
 (segment (start 19.5 11) (end 19.5 6) (width 0.2) (layer "F.Cu") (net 14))
 (segment (start 15 15.5) (end 19.5 11) (width 0.2) (layer "F.Cu") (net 14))
 (segment (start 20.5 6) (end 21.5 6) (width 0.2) (layer "F.Cu") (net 17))
 (segment (start 7 16.7) (end 7 17.2) (width 0.2) (layer "F.Cu") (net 3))
 (segment (start 6.7 16.4) (end 7 16.7) (width 0.2) (layer "F.Cu") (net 3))
 (segment (start 7 17.2) (end 7 18) (width 0.2) (layer "F.Cu") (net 3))
 (segment (start 8.95 17.25) (end 8.95 16.65) (width 0.2) (layer "F.Cu") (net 3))
 (segment (start 9.5 20.45) (end 9.125 20.65) (width 0.2) (layer "F.Cu") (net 3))
 (segment (start 8.95 16.575) (end 8.95 16.6) (width 0.2) (layer "F.Cu") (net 3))
 (segment (start 9.5 20) (end 9.5 20.45) (width 0.2) (layer "F.Cu") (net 3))
 (segment (start 7.5 37) (end 7.5 22) (width 0.2) (layer "F.Cu") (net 3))
 (segment (start 7 17.2) (end 7.05 17.25) (width 0.2) (layer "F.Cu") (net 3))
 (segment (start 7.5 22) (end 9.5 20) (width 0.2) (layer "F.Cu") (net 3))
 (via (at 6.7 16.4) (size 0.6) (drill 0.3) (layers "F.Cu" "B.Cu") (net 3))
 (via (at 9.125 20.65) (size 0.6) (drill 0.3) (layers "F.Cu" "B.Cu") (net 3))
 (via (at 8.95 16.575) (size 0.6) (drill 0.3) (layers "F.Cu" "B.Cu") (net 3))
 (segment (start 9.2 16.8) (end 9 16.6) (width 0.2) (layer "B.Cu") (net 3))
 (segment (start 7.1 16.8) (end 6.7 16.4) (width 0.2) (layer "B.Cu") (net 3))
 (segment (start 9.2 20.8) (end 9.2 16.8) (width 0.2) (layer "B.Cu") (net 3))
 (segment (start 9 16.8) (end 7.1 16.8) (width 0.2) (layer "B.Cu") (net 3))
 (segment (start 5.6 19.2) (end 5.6 33.1) (width 0.2) (layer "F.Cu") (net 16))
 (segment (start 5.6 33.1) (end 1.7 37) (width 0.2) (layer "F.Cu") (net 16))
 (segment (start 4.8 18.4) (end 5.6 19.2) (width 0.2) (layer "F.Cu") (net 16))
 (segment (start 4.8 18.2) (end 4.8 18.4) (width 0.2) (layer "F.Cu") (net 16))
 (segment (start 19.1 5.3) (end 22.9 5.3) (width 0.2) (layer "F.Cu") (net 15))
 (segment (start 22.9 5.3) (end 34 16.4) (width 0.2) (layer "F.Cu") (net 15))
 (segment (start 18.8 9.5) (end 18.8 5.6) (width 0.2) (layer "F.Cu") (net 15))
 (segment (start 34.6 18.2) (end 35.6 18.2) (width 0.2) (layer "F.Cu") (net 15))
 (segment (start 35.6 18.2) (end 38.5 21.1) (width 0.2) (layer "F.Cu") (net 15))
 (segment (start 18.8 5.6) (end 19.1 5.3) (width 0.2) (layer "F.Cu") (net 15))
 (segment (start 38.5 21.1) (end 38.5 25) (width 0.2) (layer "F.Cu") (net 15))
 (segment (start 34 16.4) (end 34 17.6) (width 0.2) (layer "F.Cu") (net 15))
 (segment (start 34 17.6) (end 34.6 18.2) (width 0.2) (layer "F.Cu") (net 15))
 (segment (start 15.5 12.8) (end 18.8 9.5) (width 0.2) (layer "F.Cu") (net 15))
 (segment (start 35.8 29.6) (end 35.2 30.2) (width 0.2) (layer "F.Cu") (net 1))
 (segment (start 41.4 29.6) (end 35.8 29.6) (width 0.2) (layer "F.Cu") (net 1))
 (segment (start 35.2 30.2) (end 17.9 30.2) (width 0.2) (layer "F.Cu") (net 1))
 (segment (start 46 25) (end 41.4 29.6) (width 0.2) (layer "F.Cu") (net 1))
 (segment (start 17.9 30.2) (end 15.1 33) (width 0.2) (layer "F.Cu") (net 1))
 (segment (start 45.1 29.1) (end 46 30) (width 0.2) (layer "F.Cu") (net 12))
 (segment (start 43.9 29.1) (end 45.1 29.1) (width 0.2) (layer "F.Cu") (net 12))
 (segment (start 40 33) (end 43.9 29.1) (width 0.2) (layer "F.Cu") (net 12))
 (segment (start 34.9 33) (end 40 33) (width 0.2) (layer "F.Cu") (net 12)))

